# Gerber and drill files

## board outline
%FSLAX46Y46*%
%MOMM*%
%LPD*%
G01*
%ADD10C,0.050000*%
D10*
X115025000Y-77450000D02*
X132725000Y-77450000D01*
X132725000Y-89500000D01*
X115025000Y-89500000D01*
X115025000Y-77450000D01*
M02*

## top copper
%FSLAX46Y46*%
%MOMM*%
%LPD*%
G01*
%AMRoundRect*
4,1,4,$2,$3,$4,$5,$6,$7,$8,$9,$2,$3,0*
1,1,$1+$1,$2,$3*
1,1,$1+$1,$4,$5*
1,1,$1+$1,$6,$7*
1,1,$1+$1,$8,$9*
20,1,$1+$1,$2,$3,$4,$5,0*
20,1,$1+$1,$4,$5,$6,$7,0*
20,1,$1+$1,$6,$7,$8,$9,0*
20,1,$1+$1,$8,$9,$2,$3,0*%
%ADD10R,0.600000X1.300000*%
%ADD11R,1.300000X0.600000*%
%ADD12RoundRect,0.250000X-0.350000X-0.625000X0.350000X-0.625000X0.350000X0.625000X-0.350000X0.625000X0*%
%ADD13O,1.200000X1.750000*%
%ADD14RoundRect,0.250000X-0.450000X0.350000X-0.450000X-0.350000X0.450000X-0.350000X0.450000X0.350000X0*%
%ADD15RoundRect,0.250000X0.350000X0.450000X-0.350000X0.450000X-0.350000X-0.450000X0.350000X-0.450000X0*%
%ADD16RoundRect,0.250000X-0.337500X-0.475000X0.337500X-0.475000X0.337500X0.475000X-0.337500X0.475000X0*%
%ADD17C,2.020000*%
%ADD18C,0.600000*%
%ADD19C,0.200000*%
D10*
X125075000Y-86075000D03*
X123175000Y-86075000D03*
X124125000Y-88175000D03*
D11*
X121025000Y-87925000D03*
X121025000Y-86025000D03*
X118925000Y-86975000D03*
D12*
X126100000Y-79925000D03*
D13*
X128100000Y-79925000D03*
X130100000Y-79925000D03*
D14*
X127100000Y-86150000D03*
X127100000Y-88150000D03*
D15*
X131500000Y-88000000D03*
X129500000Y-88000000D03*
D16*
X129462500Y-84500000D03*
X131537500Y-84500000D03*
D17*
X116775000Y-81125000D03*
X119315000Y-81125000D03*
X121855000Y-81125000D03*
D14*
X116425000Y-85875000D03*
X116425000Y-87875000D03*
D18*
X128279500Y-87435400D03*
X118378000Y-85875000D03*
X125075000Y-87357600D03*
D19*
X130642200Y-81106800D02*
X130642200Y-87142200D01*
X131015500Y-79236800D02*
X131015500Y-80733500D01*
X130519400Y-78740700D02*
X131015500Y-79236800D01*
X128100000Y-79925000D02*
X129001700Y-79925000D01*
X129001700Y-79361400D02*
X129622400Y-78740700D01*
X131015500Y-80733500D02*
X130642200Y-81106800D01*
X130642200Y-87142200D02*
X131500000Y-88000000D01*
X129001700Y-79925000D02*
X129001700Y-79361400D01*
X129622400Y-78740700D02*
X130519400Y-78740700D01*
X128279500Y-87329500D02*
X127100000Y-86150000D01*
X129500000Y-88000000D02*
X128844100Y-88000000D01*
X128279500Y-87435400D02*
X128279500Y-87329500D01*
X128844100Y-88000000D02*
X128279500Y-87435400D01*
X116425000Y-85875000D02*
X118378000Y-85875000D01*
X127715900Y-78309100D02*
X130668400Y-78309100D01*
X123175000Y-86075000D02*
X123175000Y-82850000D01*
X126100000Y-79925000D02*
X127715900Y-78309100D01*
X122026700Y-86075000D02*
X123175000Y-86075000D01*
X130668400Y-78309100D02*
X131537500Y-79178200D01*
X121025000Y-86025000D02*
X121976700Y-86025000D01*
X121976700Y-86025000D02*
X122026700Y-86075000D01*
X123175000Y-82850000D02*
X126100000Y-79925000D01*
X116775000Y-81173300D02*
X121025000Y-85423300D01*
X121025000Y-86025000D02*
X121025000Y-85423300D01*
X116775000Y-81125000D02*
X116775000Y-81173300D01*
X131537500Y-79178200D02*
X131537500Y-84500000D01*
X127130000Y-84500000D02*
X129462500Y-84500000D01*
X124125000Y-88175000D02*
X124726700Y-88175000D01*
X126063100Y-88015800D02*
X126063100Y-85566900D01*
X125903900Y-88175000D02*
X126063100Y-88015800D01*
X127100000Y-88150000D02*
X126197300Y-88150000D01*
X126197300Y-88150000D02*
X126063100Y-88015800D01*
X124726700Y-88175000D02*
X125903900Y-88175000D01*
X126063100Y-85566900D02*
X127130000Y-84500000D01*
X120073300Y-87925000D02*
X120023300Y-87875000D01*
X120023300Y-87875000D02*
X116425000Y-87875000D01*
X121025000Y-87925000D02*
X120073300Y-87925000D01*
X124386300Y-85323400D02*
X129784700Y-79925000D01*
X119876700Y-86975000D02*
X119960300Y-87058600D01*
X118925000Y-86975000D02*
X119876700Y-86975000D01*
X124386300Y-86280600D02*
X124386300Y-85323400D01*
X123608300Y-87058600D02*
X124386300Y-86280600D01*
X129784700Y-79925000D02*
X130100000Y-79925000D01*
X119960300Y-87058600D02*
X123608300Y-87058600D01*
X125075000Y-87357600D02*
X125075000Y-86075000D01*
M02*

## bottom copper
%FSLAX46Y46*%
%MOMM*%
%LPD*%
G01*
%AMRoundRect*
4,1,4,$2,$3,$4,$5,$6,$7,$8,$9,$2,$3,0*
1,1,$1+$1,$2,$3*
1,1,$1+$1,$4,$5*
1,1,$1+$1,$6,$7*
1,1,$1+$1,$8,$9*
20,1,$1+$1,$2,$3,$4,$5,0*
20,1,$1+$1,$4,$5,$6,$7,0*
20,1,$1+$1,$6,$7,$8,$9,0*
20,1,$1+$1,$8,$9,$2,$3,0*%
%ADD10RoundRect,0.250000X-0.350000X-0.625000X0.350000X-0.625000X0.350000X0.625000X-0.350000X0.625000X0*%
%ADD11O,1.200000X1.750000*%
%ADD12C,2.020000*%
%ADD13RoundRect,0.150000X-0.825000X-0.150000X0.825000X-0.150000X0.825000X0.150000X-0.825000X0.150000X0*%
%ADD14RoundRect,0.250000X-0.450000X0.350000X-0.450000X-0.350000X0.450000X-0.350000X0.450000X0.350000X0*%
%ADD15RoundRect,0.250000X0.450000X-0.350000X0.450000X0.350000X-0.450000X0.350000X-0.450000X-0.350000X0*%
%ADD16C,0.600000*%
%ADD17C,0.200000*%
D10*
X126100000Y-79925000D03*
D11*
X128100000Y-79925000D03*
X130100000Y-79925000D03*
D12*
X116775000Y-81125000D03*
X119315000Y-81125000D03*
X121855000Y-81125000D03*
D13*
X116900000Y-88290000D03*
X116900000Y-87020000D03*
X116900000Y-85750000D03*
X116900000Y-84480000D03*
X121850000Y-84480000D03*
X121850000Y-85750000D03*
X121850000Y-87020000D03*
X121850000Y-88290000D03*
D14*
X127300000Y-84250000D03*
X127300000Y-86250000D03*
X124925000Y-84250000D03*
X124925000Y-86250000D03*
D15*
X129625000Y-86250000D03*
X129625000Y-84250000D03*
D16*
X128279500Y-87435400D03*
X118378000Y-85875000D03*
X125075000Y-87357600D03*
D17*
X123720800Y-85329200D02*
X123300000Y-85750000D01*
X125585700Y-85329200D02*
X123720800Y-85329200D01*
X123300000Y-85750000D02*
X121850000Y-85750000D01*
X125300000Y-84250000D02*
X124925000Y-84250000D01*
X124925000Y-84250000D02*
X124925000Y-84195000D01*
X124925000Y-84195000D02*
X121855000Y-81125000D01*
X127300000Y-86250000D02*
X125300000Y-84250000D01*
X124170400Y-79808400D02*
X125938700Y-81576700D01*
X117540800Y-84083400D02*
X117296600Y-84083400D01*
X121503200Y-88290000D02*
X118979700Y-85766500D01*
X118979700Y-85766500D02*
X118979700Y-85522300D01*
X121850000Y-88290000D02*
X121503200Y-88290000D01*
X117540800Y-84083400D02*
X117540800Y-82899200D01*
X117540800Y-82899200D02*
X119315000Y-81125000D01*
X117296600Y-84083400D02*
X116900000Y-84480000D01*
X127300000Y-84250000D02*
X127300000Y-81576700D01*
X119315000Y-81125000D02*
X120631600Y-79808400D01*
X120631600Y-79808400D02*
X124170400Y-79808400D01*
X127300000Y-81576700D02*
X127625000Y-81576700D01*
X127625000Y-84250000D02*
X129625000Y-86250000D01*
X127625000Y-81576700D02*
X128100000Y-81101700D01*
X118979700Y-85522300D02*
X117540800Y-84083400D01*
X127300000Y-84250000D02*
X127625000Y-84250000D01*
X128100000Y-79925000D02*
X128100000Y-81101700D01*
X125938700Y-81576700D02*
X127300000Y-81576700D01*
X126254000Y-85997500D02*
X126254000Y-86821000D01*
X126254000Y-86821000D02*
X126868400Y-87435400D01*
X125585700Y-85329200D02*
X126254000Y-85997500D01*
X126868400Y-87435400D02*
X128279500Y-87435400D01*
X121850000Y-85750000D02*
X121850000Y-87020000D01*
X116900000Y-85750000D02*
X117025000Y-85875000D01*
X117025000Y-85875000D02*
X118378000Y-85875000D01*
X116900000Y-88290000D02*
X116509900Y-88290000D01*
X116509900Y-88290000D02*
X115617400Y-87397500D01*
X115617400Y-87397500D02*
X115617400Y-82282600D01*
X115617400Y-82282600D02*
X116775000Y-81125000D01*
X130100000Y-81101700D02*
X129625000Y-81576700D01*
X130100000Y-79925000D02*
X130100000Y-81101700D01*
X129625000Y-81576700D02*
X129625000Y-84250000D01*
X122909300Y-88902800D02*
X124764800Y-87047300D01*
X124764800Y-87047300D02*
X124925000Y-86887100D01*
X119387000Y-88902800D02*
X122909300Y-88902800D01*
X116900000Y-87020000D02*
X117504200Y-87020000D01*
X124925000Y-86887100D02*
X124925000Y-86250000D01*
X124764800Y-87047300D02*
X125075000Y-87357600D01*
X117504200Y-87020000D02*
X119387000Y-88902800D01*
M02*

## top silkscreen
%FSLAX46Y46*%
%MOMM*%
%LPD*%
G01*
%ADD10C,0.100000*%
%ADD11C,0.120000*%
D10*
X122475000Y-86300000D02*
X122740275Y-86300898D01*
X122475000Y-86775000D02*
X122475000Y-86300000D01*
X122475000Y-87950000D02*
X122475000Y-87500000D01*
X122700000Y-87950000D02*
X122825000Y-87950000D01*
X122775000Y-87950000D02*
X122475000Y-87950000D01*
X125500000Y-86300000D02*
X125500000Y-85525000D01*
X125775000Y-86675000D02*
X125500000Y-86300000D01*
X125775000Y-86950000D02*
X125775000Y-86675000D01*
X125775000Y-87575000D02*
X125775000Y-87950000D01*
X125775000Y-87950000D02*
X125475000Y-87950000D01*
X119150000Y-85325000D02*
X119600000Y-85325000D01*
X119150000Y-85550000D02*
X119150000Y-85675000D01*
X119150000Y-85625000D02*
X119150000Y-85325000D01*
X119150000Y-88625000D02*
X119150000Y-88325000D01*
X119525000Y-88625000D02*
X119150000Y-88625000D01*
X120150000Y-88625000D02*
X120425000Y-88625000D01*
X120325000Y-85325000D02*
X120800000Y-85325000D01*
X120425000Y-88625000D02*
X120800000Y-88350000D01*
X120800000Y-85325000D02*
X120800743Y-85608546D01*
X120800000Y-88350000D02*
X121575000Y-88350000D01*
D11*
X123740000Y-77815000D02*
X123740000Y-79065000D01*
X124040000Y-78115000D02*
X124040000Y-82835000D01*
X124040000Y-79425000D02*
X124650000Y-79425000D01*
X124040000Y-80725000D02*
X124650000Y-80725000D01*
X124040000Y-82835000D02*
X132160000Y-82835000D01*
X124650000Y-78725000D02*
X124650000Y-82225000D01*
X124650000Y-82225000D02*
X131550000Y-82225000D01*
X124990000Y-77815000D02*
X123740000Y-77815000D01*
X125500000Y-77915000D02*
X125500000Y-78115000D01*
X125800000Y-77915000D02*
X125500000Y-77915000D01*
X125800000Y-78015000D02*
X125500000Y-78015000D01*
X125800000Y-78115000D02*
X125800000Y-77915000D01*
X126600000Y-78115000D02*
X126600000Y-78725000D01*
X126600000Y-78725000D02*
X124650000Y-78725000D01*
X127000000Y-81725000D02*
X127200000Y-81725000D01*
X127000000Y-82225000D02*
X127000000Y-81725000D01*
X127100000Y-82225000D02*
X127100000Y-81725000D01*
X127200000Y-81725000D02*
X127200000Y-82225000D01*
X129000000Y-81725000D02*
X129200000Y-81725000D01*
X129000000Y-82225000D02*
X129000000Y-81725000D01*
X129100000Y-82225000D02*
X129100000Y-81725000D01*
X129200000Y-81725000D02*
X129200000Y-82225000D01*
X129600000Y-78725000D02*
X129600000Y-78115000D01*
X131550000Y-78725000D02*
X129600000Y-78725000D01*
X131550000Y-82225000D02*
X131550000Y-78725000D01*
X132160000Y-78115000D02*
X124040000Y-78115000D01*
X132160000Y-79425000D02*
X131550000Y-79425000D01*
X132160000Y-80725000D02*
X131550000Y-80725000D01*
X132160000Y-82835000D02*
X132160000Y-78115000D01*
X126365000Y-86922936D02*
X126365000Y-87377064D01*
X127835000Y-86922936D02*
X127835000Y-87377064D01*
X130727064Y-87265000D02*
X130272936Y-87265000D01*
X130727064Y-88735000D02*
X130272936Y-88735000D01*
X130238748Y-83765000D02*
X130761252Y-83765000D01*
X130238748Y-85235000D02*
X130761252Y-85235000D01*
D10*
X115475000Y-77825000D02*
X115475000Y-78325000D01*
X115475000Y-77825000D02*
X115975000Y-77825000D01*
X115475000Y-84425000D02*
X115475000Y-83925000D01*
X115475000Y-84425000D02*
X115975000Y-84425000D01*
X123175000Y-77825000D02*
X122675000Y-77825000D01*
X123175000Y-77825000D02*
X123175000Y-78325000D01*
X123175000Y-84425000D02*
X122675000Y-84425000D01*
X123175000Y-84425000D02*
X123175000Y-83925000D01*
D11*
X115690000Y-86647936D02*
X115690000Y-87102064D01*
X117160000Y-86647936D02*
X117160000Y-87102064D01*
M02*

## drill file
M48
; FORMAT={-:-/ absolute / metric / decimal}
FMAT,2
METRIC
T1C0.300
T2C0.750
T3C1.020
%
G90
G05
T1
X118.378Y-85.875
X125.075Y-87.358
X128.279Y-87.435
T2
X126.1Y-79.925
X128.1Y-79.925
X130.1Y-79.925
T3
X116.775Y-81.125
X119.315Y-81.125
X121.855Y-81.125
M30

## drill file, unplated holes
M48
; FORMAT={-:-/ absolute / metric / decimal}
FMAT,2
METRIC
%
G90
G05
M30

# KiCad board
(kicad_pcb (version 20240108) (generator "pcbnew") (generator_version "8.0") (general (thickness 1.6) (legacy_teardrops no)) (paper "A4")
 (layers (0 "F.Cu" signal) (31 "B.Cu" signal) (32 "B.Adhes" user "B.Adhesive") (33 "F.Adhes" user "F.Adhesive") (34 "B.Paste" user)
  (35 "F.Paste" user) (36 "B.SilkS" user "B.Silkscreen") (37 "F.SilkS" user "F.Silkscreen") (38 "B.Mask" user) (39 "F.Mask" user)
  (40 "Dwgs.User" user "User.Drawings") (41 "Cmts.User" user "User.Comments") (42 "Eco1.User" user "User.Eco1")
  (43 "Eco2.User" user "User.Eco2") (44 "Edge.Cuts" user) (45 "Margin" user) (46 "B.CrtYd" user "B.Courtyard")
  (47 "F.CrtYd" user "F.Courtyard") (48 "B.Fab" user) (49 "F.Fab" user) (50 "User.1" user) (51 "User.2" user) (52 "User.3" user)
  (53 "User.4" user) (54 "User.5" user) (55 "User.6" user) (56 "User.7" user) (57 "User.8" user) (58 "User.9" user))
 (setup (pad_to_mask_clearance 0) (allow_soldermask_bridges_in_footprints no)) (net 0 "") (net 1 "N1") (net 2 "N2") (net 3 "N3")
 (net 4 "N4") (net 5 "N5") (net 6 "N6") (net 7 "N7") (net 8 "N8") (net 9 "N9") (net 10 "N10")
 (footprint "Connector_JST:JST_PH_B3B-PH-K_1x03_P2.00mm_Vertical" (layer "F.Cu") (at 126.1 79.925)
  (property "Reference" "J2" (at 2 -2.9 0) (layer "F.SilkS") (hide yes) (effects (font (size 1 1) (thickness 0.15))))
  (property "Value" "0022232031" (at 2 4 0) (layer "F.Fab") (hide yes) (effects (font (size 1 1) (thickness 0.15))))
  (fp_line (start -2.36 -2.11) (end -2.36 -0.86) (stroke (width 0.12) (type solid)) (layer "F.SilkS"))
  (fp_line (start -2.06 -1.81) (end -2.06 2.91) (stroke (width 0.12) (type solid)) (layer "F.SilkS"))
  (fp_line (start -2.06 -0.5) (end -1.45 -0.5) (stroke (width 0.12) (type solid)) (layer "F.SilkS"))
  (fp_line (start -2.06 0.8) (end -1.45 0.8) (stroke (width 0.12) (type solid)) (layer "F.SilkS"))
  (fp_line (start -2.06 2.91) (end 6.06 2.91) (stroke (width 0.12) (type solid)) (layer "F.SilkS"))
  (fp_line (start -1.45 -1.2) (end -1.45 2.3) (stroke (width 0.12) (type solid)) (layer "F.SilkS"))
  (fp_line (start -1.45 2.3) (end 5.45 2.3) (stroke (width 0.12) (type solid)) (layer "F.SilkS"))
  (fp_line (start -1.11 -2.11) (end -2.36 -2.11) (stroke (width 0.12) (type solid)) (layer "F.SilkS"))
  (fp_line (start -0.6 -2.01) (end -0.6 -1.81) (stroke (width 0.12) (type solid)) (layer "F.SilkS"))
  (fp_line (start -0.3 -2.01) (end -0.6 -2.01) (stroke (width 0.12) (type solid)) (layer "F.SilkS"))
  (fp_line (start -0.3 -1.91) (end -0.6 -1.91) (stroke (width 0.12) (type solid)) (layer "F.SilkS"))
  (fp_line (start -0.3 -1.81) (end -0.3 -2.01) (stroke (width 0.12) (type solid)) (layer "F.SilkS"))
  (fp_line (start 0.5 -1.81) (end 0.5 -1.2) (stroke (width 0.12) (type solid)) (layer "F.SilkS"))
  (fp_line (start 0.5 -1.2) (end -1.45 -1.2) (stroke (width 0.12) (type solid)) (layer "F.SilkS"))
  (fp_line (start 0.9 1.8) (end 1.1 1.8) (stroke (width 0.12) (type solid)) (layer "F.SilkS"))
  (fp_line (start 0.9 2.3) (end 0.9 1.8) (stroke (width 0.12) (type solid)) (layer "F.SilkS"))
  (fp_line (start 1 2.3) (end 1 1.8) (stroke (width 0.12) (type solid)) (layer "F.SilkS"))
  (fp_line (start 1.1 1.8) (end 1.1 2.3) (stroke (width 0.12) (type solid)) (layer "F.SilkS"))
  (fp_line (start 2.9 1.8) (end 3.1 1.8) (stroke (width 0.12) (type solid)) (layer "F.SilkS"))
  (fp_line (start 2.9 2.3) (end 2.9 1.8) (stroke (width 0.12) (type solid)) (layer "F.SilkS"))
  (fp_line (start 3 2.3) (end 3 1.8) (stroke (width 0.12) (type solid)) (layer "F.SilkS"))
  (fp_line (start 3.1 1.8) (end 3.1 2.3) (stroke (width 0.12) (type solid)) (layer "F.SilkS"))
  (fp_line (start 3.5 -1.2) (end 3.5 -1.81) (stroke (width 0.12) (type solid)) (layer "F.SilkS"))
  (fp_line (start 5.45 -1.2) (end 3.5 -1.2) (stroke (width 0.12) (type solid)) (layer "F.SilkS"))
  (fp_line (start 5.45 2.3) (end 5.45 -1.2) (stroke (width 0.12) (type solid)) (layer "F.SilkS"))
  (fp_line (start 6.06 -1.81) (end -2.06 -1.81) (stroke (width 0.12) (type solid)) (layer "F.SilkS"))
  (fp_line (start 6.06 -0.5) (end 5.45 -0.5) (stroke (width 0.12) (type solid)) (layer "F.SilkS"))
  (fp_line (start 6.06 0.8) (end 5.45 0.8) (stroke (width 0.12) (type solid)) (layer "F.SilkS"))
  (fp_line (start 6.06 2.91) (end 6.06 -1.81) (stroke (width 0.12) (type solid)) (layer "F.SilkS"))
  (pad "1" thru_hole roundrect (at 0 0) (size 1.2 1.75) (drill 0.75) (layers "*.Cu" "*.Mask") (remove_unused_layers no)
   (roundrect_rratio 0.208333) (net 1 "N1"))
  (pad "2" thru_hole oval (at 2 0) (size 1.2 1.75) (drill 0.75) (layers "*.Cu" "*.Mask") (remove_unused_layers no) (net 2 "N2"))
  (pad "3" thru_hole oval (at 4 0) (size 1.2 1.75) (drill 0.75) (layers "*.Cu" "*.Mask") (remove_unused_layers no) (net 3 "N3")))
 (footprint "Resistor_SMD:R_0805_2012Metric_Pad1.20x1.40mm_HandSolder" (layer "F.Cu") (at 127.1 87.15 -90)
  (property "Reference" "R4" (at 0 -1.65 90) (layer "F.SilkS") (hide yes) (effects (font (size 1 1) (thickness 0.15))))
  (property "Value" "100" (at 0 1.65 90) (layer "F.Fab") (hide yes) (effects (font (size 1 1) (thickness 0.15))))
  (fp_line (start -0.227064 0.735) (end 0.227064 0.735) (stroke (width 0.12) (type solid)) (layer "F.SilkS"))
  (fp_line (start -0.227064 -0.735) (end 0.227064 -0.735) (stroke (width 0.12) (type solid)) (layer "F.SilkS"))
  (pad "1" smd roundrect (at -1 0 270) (size 1.2 1.4) (layers "F.Cu" "F.Paste" "F.Mask") (roundrect_rratio 0.208333) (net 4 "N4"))
  (pad "2" smd roundrect (at 1 0 270) (size 1.2 1.4) (layers "F.Cu" "F.Paste" "F.Mask") (roundrect_rratio 0.208333) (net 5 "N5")))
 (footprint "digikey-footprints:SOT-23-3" (layer "F.Cu") (at 119.975 86.975 180)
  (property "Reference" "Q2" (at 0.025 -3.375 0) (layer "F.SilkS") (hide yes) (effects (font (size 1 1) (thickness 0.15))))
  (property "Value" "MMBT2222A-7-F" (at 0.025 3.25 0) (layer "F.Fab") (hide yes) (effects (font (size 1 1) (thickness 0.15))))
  (fp_line (start 0.825 1.65) (end 0.375 1.65) (stroke (width 0.1) (type solid)) (layer "F.SilkS"))
  (fp_line (start 0.825 1.425) (end 0.825 1.3) (stroke (width 0.1) (type solid)) (layer "F.SilkS"))
  (fp_line (start 0.825 1.35) (end 0.825 1.65) (stroke (width 0.1) (type solid)) (layer "F.SilkS"))
  (fp_line (start 0.825 -1.65) (end 0.825 -1.35) (stroke (width 0.1) (type solid)) (layer "F.SilkS"))
  (fp_line (start 0.45 -1.65) (end 0.825 -1.65) (stroke (width 0.1) (type solid)) (layer "F.SilkS"))
  (fp_line (start -0.175 -1.65) (end -0.45 -1.65) (stroke (width 0.1) (type solid)) (layer "F.SilkS"))
  (fp_line (start -0.35 1.65) (end -0.825 1.65) (stroke (width 0.1) (type solid)) (layer "F.SilkS"))
  (fp_line (start -0.45 -1.65) (end -0.825 -1.375) (stroke (width 0.1) (type solid)) (layer "F.SilkS"))
  (fp_line (start -0.825 1.65) (end -0.825743 1.366454) (stroke (width 0.1) (type solid)) (layer "F.SilkS"))
  (fp_line (start -0.825 -1.375) (end -1.6 -1.375) (stroke (width 0.1) (type solid)) (layer "F.SilkS"))
  (pad "1" smd rect (at -1.05 -0.95 180) (size 1.3 0.6) (layers "F.Cu" "F.Paste" "F.Mask") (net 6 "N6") (solder_mask_margin 0.07))
  (pad "2" smd rect (at -1.05 0.95 180) (size 1.3 0.6) (layers "F.Cu" "F.Paste" "F.Mask") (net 1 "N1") (solder_mask_margin 0.07))
  (pad "3" smd rect (at 1.05 0 180) (size 1.3 0.6) (layers "F.Cu" "F.Paste" "F.Mask") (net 3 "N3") (solder_mask_margin 0.07)))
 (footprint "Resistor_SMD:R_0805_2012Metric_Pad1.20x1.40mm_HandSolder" (layer "F.Cu") (at 130.5 88 180)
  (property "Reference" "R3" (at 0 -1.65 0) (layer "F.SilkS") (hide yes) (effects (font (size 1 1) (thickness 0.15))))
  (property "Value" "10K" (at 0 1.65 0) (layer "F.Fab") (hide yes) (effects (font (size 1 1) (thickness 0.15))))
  (fp_line (start -0.227064 0.735) (end 0.227064 0.735) (stroke (width 0.12) (type solid)) (layer "F.SilkS"))
  (fp_line (start -0.227064 -0.735) (end 0.227064 -0.735) (stroke (width 0.12) (type solid)) (layer "F.SilkS"))
  (pad "1" smd roundrect (at -1 0 180) (size 1.2 1.4) (layers "F.Cu" "F.Paste" "F.Mask") (roundrect_rratio 0.208333) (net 2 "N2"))
  (pad "2" smd roundrect (at 1 0 180) (size 1.2 1.4) (layers "F.Cu" "F.Paste" "F.Mask") (roundrect_rratio 0.208333) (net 4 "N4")))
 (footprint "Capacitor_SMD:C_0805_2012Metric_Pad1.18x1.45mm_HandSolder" (layer "F.Cu") (at 130.5 84.5)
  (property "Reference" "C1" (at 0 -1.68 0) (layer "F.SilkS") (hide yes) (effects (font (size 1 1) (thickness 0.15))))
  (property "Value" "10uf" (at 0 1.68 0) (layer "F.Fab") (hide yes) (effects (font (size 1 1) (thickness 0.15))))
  (fp_line (start -0.261252 -0.735) (end 0.261252 -0.735) (stroke (width 0.12) (type solid)) (layer "F.SilkS"))
  (fp_line (start -0.261252 0.735) (end 0.261252 0.735) (stroke (width 0.12) (type solid)) (layer "F.SilkS"))
  (pad "1" smd roundrect (at -1.0375 0) (size 1.175 1.45) (layers "F.Cu" "F.Paste" "F.Mask") (roundrect_rratio 0.212766) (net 5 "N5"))
  (pad "2" smd roundrect (at 1.0375 0) (size 1.175 1.45) (layers "F.Cu" "F.Paste" "F.Mask") (roundrect_rratio 0.212766) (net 1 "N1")))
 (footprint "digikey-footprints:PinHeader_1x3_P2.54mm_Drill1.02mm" (layer "F.Cu") (at 116.775 81.125)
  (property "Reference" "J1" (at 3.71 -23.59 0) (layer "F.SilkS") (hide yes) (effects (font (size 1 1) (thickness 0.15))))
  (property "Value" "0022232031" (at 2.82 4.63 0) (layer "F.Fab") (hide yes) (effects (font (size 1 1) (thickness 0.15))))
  (fp_line (start -1.3 -3.3) (end -1.3 -2.8) (stroke (width 0.1) (type solid)) (layer "F.SilkS"))
  (fp_line (start -1.3 -3.3) (end -0.8 -3.3) (stroke (width 0.1) (type solid)) (layer "F.SilkS"))
  (fp_line (start -1.3 3.3) (end -1.3 2.8) (stroke (width 0.1) (type solid)) (layer "F.SilkS"))
  (fp_line (start -1.3 3.3) (end -0.8 3.3) (stroke (width 0.1) (type solid)) (layer "F.SilkS"))
  (fp_line (start 6.4 -3.3) (end 5.9 -3.3) (stroke (width 0.1) (type solid)) (layer "F.SilkS"))
  (fp_line (start 6.4 -3.3) (end 6.4 -2.8) (stroke (width 0.1) (type solid)) (layer "F.SilkS"))
  (fp_line (start 6.4 3.3) (end 5.9 3.3) (stroke (width 0.1) (type solid)) (layer "F.SilkS"))
  (fp_line (start 6.4 3.3) (end 6.4 2.8) (stroke (width 0.1) (type solid)) (layer "F.SilkS"))
  (pad "1" thru_hole circle (at 0 0) (size 2.02 2.02) (drill 1.02) (layers "*.Cu" "*.Mask") (remove_unused_layers no) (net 1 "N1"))
  (pad "2" thru_hole circle (at 2.54 0) (size 2.02 2.02) (drill 1.02) (layers "*.Cu" "*.Mask") (remove_unused_layers no) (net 2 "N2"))
  (pad "3" thru_hole circle (at 5.08 0) (size 2.02 2.02) (drill 1.02) (layers "*.Cu" "*.Mask") (remove_unused_layers no) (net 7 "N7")))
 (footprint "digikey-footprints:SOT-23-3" (layer "F.Cu") (at 124.125 87.125 -90)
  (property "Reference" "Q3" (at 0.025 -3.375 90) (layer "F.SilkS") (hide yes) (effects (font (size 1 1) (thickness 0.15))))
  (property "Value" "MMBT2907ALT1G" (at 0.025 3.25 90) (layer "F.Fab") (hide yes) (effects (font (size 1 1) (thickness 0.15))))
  (fp_line (start -0.825 1.65) (end -0.824102 1.384725) (stroke (width 0.1) (type solid)) (layer "F.SilkS"))
  (fp_line (start -0.35 1.65) (end -0.825 1.65) (stroke (width 0.1) (type solid)) (layer "F.SilkS"))
  (fp_line (start 0.825 1.65) (end 0.375 1.65) (stroke (width 0.1) (type solid)) (layer "F.SilkS"))
  (fp_line (start 0.825 1.425) (end 0.825 1.3) (stroke (width 0.1) (type solid)) (layer "F.SilkS"))
  (fp_line (start 0.825 1.35) (end 0.825 1.65) (stroke (width 0.1) (type solid)) (layer "F.SilkS"))
  (fp_line (start -0.825 -1.375) (end -1.6 -1.375) (stroke (width 0.1) (type solid)) (layer "F.SilkS"))
  (fp_line (start -0.45 -1.65) (end -0.825 -1.375) (stroke (width 0.1) (type solid)) (layer "F.SilkS"))
  (fp_line (start -0.175 -1.65) (end -0.45 -1.65) (stroke (width 0.1) (type solid)) (layer "F.SilkS"))
  (fp_line (start 0.45 -1.65) (end 0.825 -1.65) (stroke (width 0.1) (type solid)) (layer "F.SilkS"))
  (fp_line (start 0.825 -1.65) (end 0.825 -1.35) (stroke (width 0.1) (type solid)) (layer "F.SilkS"))
  (pad "1" smd rect (at -1.05 -0.95 270) (size 1.3 0.6) (layers "F.Cu" "F.Paste" "F.Mask") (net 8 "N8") (solder_mask_margin 0.07))
  (pad "2" smd rect (at -1.05 0.95 270) (size 1.3 0.6) (layers "F.Cu" "F.Paste" "F.Mask") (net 1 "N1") (solder_mask_margin 0.07))
  (pad "3" smd rect (at 1.05 0 270) (size 1.3 0.6) (layers "F.Cu" "F.Paste" "F.Mask") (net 5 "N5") (solder_mask_margin 0.07)))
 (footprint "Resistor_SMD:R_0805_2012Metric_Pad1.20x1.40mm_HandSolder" (layer "F.Cu") (at 116.425 86.875 -90)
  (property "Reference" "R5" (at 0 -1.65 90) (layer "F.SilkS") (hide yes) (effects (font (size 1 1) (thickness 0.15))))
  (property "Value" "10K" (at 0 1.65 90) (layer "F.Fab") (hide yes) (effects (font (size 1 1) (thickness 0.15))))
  (fp_line (start -0.227064 0.735) (end 0.227064 0.735) (stroke (width 0.12) (type solid)) (layer "F.SilkS"))
  (fp_line (start -0.227064 -0.735) (end 0.227064 -0.735) (stroke (width 0.12) (type solid)) (layer "F.SilkS"))
  (pad "1" smd roundrect (at -1 0 270) (size 1.2 1.4) (layers "F.Cu" "F.Paste" "F.Mask") (roundrect_rratio 0.208333) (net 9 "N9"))
  (pad "2" smd roundrect (at 1 0 270) (size 1.2 1.4) (layers "F.Cu" "F.Paste" "F.Mask") (roundrect_rratio 0.208333) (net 6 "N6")))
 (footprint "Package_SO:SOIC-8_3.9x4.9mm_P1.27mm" (layer "B.Cu") (at 119.375 86.385)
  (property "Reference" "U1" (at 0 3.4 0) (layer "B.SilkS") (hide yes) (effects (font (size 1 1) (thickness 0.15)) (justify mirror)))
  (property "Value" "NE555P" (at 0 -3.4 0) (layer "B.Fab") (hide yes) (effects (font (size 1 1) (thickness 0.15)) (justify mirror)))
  (pad "1" smd roundrect (at -2.475 1.905) (size 1.95 0.6) (layers "B.Cu" "B.Paste" "B.Mask") (roundrect_rratio 0.25) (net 1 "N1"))
  (pad "2" smd roundrect (at -2.475 0.635) (size 1.95 0.6) (layers "B.Cu" "B.Paste" "B.Mask") (roundrect_rratio 0.25) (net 8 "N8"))
  (pad "3" smd roundrect (at -2.475 -0.635) (size 1.95 0.6) (layers "B.Cu" "B.Paste" "B.Mask") (roundrect_rratio 0.25) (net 9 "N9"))
  (pad "4" smd roundrect (at -2.475 -1.905) (size 1.95 0.6) (layers "B.Cu" "B.Paste" "B.Mask") (roundrect_rratio 0.25) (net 2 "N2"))
  (pad "5" smd roundrect (at 2.475 -1.905) (size 1.95 0.6) (layers "B.Cu" "B.Paste" "B.Mask") (roundrect_rratio 0.25) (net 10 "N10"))
  (pad "6" smd roundrect (at 2.475 -0.635) (size 1.95 0.6) (layers "B.Cu" "B.Paste" "B.Mask") (roundrect_rratio 0.25) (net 4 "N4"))
  (pad "7" smd roundrect (at 2.475 0.635) (size 1.95 0.6) (layers "B.Cu" "B.Paste" "B.Mask") (roundrect_rratio 0.25) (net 4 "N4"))
  (pad "8" smd roundrect (at 2.475 1.905) (size 1.95 0.6) (layers "B.Cu" "B.Paste" "B.Mask") (roundrect_rratio 0.25) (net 2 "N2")))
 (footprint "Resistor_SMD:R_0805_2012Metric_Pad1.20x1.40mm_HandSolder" (layer "B.Cu") (at 127.3 85.25 -90)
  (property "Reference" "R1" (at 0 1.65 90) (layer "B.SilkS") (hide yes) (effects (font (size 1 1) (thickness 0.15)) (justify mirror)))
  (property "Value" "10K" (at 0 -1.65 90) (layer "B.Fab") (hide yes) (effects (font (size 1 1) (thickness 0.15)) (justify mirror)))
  (pad "1" smd roundrect (at -1 0 270) (size 1.2 1.4) (layers "B.Cu" "B.Paste" "B.Mask") (roundrect_rratio 0.208333) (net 2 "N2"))
  (pad "2" smd roundrect (at 1 0 270) (size 1.2 1.4) (layers "B.Cu" "B.Paste" "B.Mask") (roundrect_rratio 0.208333) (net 7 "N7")))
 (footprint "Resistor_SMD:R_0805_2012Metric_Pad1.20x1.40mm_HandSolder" (layer "B.Cu") (at 124.925 85.25 -90)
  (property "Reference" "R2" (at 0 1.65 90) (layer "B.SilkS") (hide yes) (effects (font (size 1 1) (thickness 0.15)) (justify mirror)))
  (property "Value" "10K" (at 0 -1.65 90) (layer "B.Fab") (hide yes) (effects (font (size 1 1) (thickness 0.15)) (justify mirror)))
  (pad "1" smd roundrect (at -1 0 270) (size 1.2 1.4) (layers "B.Cu" "B.Paste" "B.Mask") (roundrect_rratio 0.208333) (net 7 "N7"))
  (pad "2" smd roundrect (at 1 0 270) (size 1.2 1.4) (layers "B.Cu" "B.Paste" "B.Mask") (roundrect_rratio 0.208333) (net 8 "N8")))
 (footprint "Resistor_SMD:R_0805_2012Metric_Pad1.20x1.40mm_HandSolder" (layer "B.Cu") (at 129.625 85.25 90)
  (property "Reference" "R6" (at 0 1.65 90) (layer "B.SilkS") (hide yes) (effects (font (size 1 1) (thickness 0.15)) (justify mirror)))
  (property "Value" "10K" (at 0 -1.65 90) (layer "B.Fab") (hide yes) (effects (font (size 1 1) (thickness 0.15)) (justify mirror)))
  (pad "1" smd roundrect (at -1 0 90) (size 1.2 1.4) (layers "B.Cu" "B.Paste" "B.Mask") (roundrect_rratio 0.208333) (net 2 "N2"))
  (pad "2" smd roundrect (at 1 0 90) (size 1.2 1.4) (layers "B.Cu" "B.Paste" "B.Mask") (roundrect_rratio 0.208333) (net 3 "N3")))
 (gr_rect (start 115.025 77.45) (end 132.725 89.5) (stroke (width 0.05) (type default)) (fill none) (layer "Edge.Cuts"))
 (segment (start 125.3 84.25) (end 124.925 84.25) (width 0.2) (layer "B.Cu") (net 7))
 (segment (start 124.925 84.25) (end 124.925 84.195) (width 0.2) (layer "B.Cu") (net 7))
 (segment (start 124.925 84.195) (end 121.855 81.125) (width 0.2) (layer "B.Cu") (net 7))
 (segment (start 127.3 86.25) (end 125.3 84.25) (width 0.2) (layer "B.Cu") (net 7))
 (segment (start 130.6422 81.1068) (end 130.6422 87.1422) (width 0.2) (layer "F.Cu") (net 2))
 (segment (start 131.0155 79.2368) (end 131.0155 80.7335) (width 0.2) (layer "F.Cu") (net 2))
 (segment (start 130.5194 78.7407) (end 131.0155 79.2368) (width 0.2) (layer "F.Cu") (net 2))
 (segment (start 128.1 79.925) (end 129.0017 79.925) (width 0.2) (layer "F.Cu") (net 2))
 (segment (start 129.0017 79.3614) (end 129.6224 78.7407) (width 0.2) (layer "F.Cu") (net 2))
 (segment (start 131.0155 80.7335) (end 130.6422 81.1068) (width 0.2) (layer "F.Cu") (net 2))
 (segment (start 130.6422 87.1422) (end 131.5 88) (width 0.2) (layer "F.Cu") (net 2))
 (segment (start 129.0017 79.925) (end 129.0017 79.3614) (width 0.2) (layer "F.Cu") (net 2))
 (segment (start 129.6224 78.7407) (end 130.5194 78.7407) (width 0.2) (layer "F.Cu") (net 2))
 (segment (start 124.1704 79.8084) (end 125.9387 81.5767) (width 0.2) (layer "B.Cu") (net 2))
 (segment (start 117.5408 84.0834) (end 117.2966 84.0834) (width 0.2) (layer "B.Cu") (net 2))
 (segment (start 121.5032 88.29) (end 118.9797 85.7665) (width 0.2) (layer "B.Cu") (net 2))
 (segment (start 118.9797 85.7665) (end 118.9797 85.5223) (width 0.2) (layer "B.Cu") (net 2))
 (segment (start 121.85 88.29) (end 121.5032 88.29) (width 0.2) (layer "B.Cu") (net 2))
 (segment (start 117.5408 84.0834) (end 117.5408 82.8992) (width 0.2) (layer "B.Cu") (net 2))
 (segment (start 117.5408 82.8992) (end 119.315 81.125) (width 0.2) (layer "B.Cu") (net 2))
 (segment (start 117.2966 84.0834) (end 116.9 84.48) (width 0.2) (layer "B.Cu") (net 2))
 (segment (start 127.3 84.25) (end 127.3 81.5767) (width 0.2) (layer "B.Cu") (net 2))
 (segment (start 119.315 81.125) (end 120.6316 79.8084) (width 0.2) (layer "B.Cu") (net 2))
 (segment (start 120.6316 79.8084) (end 124.1704 79.8084) (width 0.2) (layer "B.Cu") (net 2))
 (segment (start 127.3 81.5767) (end 127.625 81.5767) (width 0.2) (layer "B.Cu") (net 2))
 (segment (start 127.625 84.25) (end 129.625 86.25) (width 0.2) (layer "B.Cu") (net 2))
 (segment (start 127.625 81.5767) (end 128.1 81.1017) (width 0.2) (layer "B.Cu") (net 2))
 (segment (start 118.9797 85.5223) (end 117.5408 84.0834) (width 0.2) (layer "B.Cu") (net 2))
 (segment (start 127.3 84.25) (end 127.625 84.25) (width 0.2) (layer "B.Cu") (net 2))
 (segment (start 128.1 79.925) (end 128.1 81.1017) (width 0.2) (layer "B.Cu") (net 2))
 (segment (start 125.9387 81.5767) (end 127.3 81.5767) (width 0.2) (layer "B.Cu") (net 2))
 (segment (start 128.2795 87.3295) (end 127.1 86.15) (width 0.2) (layer "F.Cu") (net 4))
 (segment (start 129.5 88) (end 128.8441 88) (width 0.2) (layer "F.Cu") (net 4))
 (segment (start 128.2795 87.4354) (end 128.2795 87.3295) (width 0.2) (layer "F.Cu") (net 4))
 (segment (start 128.8441 88) (end 128.2795 87.4354) (width 0.2) (layer "F.Cu") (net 4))
 (via (at 128.2795 87.4354) (size 0.6) (drill 0.3) (layers "F.Cu" "B.Cu") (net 4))
 (segment (start 126.254 85.9975) (end 126.254 86.821) (width 0.2) (layer "B.Cu") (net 4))
 (segment (start 126.254 86.821) (end 126.8684 87.4354) (width 0.2) (layer "B.Cu") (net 4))
 (segment (start 125.5857 85.3292) (end 123.7208 85.3292) (width 0.2) (layer "B.Cu") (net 4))
 (segment (start 125.5857 85.3292) (end 126.254 85.9975) (width 0.2) (layer "B.Cu") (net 4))
 (segment (start 126.8684 87.4354) (end 128.2795 87.4354) (width 0.2) (layer "B.Cu") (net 4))
 (segment (start 123.7208 85.3292) (end 123.3 85.75) (width 0.2) (layer "B.Cu") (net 4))
 (segment (start 121.85 85.75) (end 121.85 87.02) (width 0.2) (layer "B.Cu") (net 4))
 (segment (start 123.3 85.75) (end 121.85 85.75) (width 0.2) (layer "B.Cu") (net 4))
 (segment (start 116.425 85.875) (end 118.378 85.875) (width 0.2) (layer "F.Cu") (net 9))
 (via (at 118.378 85.875) (size 0.6) (drill 0.3) (layers "F.Cu" "B.Cu") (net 9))
 (segment (start 116.9 85.75) (end 117.025 85.875) (width 0.2) (layer "B.Cu") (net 9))
 (segment (start 117.025 85.875) (end 118.378 85.875) (width 0.2) (layer "B.Cu") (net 9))
 (segment (start 127.7159 78.3091) (end 130.6684 78.3091) (width 0.2) (layer "F.Cu") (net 1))
 (segment (start 123.175 86.075) (end 123.175 82.85) (width 0.2) (layer "F.Cu") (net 1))
 (segment (start 126.1 79.925) (end 127.7159 78.3091) (width 0.2) (layer "F.Cu") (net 1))
 (segment (start 122.0267 86.075) (end 123.175 86.075) (width 0.2) (layer "F.Cu") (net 1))
 (segment (start 130.6684 78.3091) (end 131.5375 79.1782) (width 0.2) (layer "F.Cu") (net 1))
 (segment (start 121.025 86.025) (end 121.9767 86.025) (width 0.2) (layer "F.Cu") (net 1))
 (segment (start 121.9767 86.025) (end 122.0267 86.075) (width 0.2) (layer "F.Cu") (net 1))
 (segment (start 123.175 82.85) (end 126.1 79.925) (width 0.2) (layer "F.Cu") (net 1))
 (segment (start 116.775 81.1733) (end 121.025 85.4233) (width 0.2) (layer "F.Cu") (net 1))
 (segment (start 121.025 86.025) (end 121.025 85.4233) (width 0.2) (layer "F.Cu") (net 1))
 (segment (start 116.775 81.125) (end 116.775 81.1733) (width 0.2) (layer "F.Cu") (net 1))
 (segment (start 131.5375 79.1782) (end 131.5375 84.5) (width 0.2) (layer "F.Cu") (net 1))
 (segment (start 116.9 88.29) (end 116.5099 88.29) (width 0.2) (layer "B.Cu") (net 1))
 (segment (start 116.5099 88.29) (end 115.6174 87.3975) (width 0.2) (layer "B.Cu") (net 1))
 (segment (start 115.6174 87.3975) (end 115.6174 82.2826) (width 0.2) (layer "B.Cu") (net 1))
 (segment (start 115.6174 82.2826) (end 116.775 81.125) (width 0.2) (layer "B.Cu") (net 1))
 (segment (start 127.13 84.5) (end 129.4625 84.5) (width 0.2) (layer "F.Cu") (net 5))
 (segment (start 124.125 88.175) (end 124.7267 88.175) (width 0.2) (layer "F.Cu") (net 5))
 (segment (start 126.0631 88.0158) (end 126.0631 85.5669) (width 0.2) (layer "F.Cu") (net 5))
 (segment (start 125.9039 88.175) (end 126.0631 88.0158) (width 0.2) (layer "F.Cu") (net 5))
 (segment (start 127.1 88.15) (end 126.1973 88.15) (width 0.2) (layer "F.Cu") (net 5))
 (segment (start 126.1973 88.15) (end 126.0631 88.0158) (width 0.2) (layer "F.Cu") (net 5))
 (segment (start 124.7267 88.175) (end 125.9039 88.175) (width 0.2) (layer "F.Cu") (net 5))
 (segment (start 126.0631 85.5669) (end 127.13 84.5) (width 0.2) (layer "F.Cu") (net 5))
 (segment (start 120.0733 87.925) (end 120.0233 87.875) (width 0.2) (layer "F.Cu") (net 6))
 (segment (start 120.0233 87.875) (end 116.425 87.875) (width 0.2) (layer "F.Cu") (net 6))
 (segment (start 121.025 87.925) (end 120.0733 87.925) (width 0.2) (layer "F.Cu") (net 6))
 (segment (start 124.3863 85.3234) (end 129.7847 79.925) (width 0.2) (layer "F.Cu") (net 3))
 (segment (start 119.8767 86.975) (end 119.9603 87.0586) (width 0.2) (layer "F.Cu") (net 3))
 (segment (start 118.925 86.975) (end 119.8767 86.975) (width 0.2) (layer "F.Cu") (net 3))
 (segment (start 124.3863 86.2806) (end 124.3863 85.3234) (width 0.2) (layer "F.Cu") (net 3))
 (segment (start 123.6083 87.0586) (end 124.3863 86.2806) (width 0.2) (layer "F.Cu") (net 3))
 (segment (start 129.7847 79.925) (end 130.1 79.925) (width 0.2) (layer "F.Cu") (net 3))
 (segment (start 119.9603 87.0586) (end 123.6083 87.0586) (width 0.2) (layer "F.Cu") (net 3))
 (segment (start 130.1 81.1017) (end 129.625 81.5767) (width 0.2) (layer "B.Cu") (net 3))
 (segment (start 130.1 79.925) (end 130.1 81.1017) (width 0.2) (layer "B.Cu") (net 3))
 (segment (start 129.625 81.5767) (end 129.625 84.25) (width 0.2) (layer "B.Cu") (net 3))
 (segment (start 125.075 87.3576) (end 125.075 86.075) (width 0.2) (layer "F.Cu") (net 8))
 (via (at 125.075 87.3576) (size 0.6) (drill 0.3) (layers "F.Cu" "B.Cu") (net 8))
 (segment (start 122.9093 88.9028) (end 124.7648 87.0473) (width 0.2) (layer "B.Cu") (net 8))
 (segment (start 124.7648 87.0473) (end 124.925 86.8871) (width 0.2) (layer "B.Cu") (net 8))
 (segment (start 119.387 88.9028) (end 122.9093 88.9028) (width 0.2) (layer "B.Cu") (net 8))
 (segment (start 116.9 87.02) (end 117.5042 87.02) (width 0.2) (layer "B.Cu") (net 8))
 (segment (start 124.925 86.8871) (end 124.925 86.25) (width 0.2) (layer "B.Cu") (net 8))
 (segment (start 124.7648 87.0473) (end 125.075 87.3576) (width 0.2) (layer "B.Cu") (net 8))
 (segment (start 117.5042 87.02) (end 119.387 88.9028) (width 0.2) (layer "B.Cu") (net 8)))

